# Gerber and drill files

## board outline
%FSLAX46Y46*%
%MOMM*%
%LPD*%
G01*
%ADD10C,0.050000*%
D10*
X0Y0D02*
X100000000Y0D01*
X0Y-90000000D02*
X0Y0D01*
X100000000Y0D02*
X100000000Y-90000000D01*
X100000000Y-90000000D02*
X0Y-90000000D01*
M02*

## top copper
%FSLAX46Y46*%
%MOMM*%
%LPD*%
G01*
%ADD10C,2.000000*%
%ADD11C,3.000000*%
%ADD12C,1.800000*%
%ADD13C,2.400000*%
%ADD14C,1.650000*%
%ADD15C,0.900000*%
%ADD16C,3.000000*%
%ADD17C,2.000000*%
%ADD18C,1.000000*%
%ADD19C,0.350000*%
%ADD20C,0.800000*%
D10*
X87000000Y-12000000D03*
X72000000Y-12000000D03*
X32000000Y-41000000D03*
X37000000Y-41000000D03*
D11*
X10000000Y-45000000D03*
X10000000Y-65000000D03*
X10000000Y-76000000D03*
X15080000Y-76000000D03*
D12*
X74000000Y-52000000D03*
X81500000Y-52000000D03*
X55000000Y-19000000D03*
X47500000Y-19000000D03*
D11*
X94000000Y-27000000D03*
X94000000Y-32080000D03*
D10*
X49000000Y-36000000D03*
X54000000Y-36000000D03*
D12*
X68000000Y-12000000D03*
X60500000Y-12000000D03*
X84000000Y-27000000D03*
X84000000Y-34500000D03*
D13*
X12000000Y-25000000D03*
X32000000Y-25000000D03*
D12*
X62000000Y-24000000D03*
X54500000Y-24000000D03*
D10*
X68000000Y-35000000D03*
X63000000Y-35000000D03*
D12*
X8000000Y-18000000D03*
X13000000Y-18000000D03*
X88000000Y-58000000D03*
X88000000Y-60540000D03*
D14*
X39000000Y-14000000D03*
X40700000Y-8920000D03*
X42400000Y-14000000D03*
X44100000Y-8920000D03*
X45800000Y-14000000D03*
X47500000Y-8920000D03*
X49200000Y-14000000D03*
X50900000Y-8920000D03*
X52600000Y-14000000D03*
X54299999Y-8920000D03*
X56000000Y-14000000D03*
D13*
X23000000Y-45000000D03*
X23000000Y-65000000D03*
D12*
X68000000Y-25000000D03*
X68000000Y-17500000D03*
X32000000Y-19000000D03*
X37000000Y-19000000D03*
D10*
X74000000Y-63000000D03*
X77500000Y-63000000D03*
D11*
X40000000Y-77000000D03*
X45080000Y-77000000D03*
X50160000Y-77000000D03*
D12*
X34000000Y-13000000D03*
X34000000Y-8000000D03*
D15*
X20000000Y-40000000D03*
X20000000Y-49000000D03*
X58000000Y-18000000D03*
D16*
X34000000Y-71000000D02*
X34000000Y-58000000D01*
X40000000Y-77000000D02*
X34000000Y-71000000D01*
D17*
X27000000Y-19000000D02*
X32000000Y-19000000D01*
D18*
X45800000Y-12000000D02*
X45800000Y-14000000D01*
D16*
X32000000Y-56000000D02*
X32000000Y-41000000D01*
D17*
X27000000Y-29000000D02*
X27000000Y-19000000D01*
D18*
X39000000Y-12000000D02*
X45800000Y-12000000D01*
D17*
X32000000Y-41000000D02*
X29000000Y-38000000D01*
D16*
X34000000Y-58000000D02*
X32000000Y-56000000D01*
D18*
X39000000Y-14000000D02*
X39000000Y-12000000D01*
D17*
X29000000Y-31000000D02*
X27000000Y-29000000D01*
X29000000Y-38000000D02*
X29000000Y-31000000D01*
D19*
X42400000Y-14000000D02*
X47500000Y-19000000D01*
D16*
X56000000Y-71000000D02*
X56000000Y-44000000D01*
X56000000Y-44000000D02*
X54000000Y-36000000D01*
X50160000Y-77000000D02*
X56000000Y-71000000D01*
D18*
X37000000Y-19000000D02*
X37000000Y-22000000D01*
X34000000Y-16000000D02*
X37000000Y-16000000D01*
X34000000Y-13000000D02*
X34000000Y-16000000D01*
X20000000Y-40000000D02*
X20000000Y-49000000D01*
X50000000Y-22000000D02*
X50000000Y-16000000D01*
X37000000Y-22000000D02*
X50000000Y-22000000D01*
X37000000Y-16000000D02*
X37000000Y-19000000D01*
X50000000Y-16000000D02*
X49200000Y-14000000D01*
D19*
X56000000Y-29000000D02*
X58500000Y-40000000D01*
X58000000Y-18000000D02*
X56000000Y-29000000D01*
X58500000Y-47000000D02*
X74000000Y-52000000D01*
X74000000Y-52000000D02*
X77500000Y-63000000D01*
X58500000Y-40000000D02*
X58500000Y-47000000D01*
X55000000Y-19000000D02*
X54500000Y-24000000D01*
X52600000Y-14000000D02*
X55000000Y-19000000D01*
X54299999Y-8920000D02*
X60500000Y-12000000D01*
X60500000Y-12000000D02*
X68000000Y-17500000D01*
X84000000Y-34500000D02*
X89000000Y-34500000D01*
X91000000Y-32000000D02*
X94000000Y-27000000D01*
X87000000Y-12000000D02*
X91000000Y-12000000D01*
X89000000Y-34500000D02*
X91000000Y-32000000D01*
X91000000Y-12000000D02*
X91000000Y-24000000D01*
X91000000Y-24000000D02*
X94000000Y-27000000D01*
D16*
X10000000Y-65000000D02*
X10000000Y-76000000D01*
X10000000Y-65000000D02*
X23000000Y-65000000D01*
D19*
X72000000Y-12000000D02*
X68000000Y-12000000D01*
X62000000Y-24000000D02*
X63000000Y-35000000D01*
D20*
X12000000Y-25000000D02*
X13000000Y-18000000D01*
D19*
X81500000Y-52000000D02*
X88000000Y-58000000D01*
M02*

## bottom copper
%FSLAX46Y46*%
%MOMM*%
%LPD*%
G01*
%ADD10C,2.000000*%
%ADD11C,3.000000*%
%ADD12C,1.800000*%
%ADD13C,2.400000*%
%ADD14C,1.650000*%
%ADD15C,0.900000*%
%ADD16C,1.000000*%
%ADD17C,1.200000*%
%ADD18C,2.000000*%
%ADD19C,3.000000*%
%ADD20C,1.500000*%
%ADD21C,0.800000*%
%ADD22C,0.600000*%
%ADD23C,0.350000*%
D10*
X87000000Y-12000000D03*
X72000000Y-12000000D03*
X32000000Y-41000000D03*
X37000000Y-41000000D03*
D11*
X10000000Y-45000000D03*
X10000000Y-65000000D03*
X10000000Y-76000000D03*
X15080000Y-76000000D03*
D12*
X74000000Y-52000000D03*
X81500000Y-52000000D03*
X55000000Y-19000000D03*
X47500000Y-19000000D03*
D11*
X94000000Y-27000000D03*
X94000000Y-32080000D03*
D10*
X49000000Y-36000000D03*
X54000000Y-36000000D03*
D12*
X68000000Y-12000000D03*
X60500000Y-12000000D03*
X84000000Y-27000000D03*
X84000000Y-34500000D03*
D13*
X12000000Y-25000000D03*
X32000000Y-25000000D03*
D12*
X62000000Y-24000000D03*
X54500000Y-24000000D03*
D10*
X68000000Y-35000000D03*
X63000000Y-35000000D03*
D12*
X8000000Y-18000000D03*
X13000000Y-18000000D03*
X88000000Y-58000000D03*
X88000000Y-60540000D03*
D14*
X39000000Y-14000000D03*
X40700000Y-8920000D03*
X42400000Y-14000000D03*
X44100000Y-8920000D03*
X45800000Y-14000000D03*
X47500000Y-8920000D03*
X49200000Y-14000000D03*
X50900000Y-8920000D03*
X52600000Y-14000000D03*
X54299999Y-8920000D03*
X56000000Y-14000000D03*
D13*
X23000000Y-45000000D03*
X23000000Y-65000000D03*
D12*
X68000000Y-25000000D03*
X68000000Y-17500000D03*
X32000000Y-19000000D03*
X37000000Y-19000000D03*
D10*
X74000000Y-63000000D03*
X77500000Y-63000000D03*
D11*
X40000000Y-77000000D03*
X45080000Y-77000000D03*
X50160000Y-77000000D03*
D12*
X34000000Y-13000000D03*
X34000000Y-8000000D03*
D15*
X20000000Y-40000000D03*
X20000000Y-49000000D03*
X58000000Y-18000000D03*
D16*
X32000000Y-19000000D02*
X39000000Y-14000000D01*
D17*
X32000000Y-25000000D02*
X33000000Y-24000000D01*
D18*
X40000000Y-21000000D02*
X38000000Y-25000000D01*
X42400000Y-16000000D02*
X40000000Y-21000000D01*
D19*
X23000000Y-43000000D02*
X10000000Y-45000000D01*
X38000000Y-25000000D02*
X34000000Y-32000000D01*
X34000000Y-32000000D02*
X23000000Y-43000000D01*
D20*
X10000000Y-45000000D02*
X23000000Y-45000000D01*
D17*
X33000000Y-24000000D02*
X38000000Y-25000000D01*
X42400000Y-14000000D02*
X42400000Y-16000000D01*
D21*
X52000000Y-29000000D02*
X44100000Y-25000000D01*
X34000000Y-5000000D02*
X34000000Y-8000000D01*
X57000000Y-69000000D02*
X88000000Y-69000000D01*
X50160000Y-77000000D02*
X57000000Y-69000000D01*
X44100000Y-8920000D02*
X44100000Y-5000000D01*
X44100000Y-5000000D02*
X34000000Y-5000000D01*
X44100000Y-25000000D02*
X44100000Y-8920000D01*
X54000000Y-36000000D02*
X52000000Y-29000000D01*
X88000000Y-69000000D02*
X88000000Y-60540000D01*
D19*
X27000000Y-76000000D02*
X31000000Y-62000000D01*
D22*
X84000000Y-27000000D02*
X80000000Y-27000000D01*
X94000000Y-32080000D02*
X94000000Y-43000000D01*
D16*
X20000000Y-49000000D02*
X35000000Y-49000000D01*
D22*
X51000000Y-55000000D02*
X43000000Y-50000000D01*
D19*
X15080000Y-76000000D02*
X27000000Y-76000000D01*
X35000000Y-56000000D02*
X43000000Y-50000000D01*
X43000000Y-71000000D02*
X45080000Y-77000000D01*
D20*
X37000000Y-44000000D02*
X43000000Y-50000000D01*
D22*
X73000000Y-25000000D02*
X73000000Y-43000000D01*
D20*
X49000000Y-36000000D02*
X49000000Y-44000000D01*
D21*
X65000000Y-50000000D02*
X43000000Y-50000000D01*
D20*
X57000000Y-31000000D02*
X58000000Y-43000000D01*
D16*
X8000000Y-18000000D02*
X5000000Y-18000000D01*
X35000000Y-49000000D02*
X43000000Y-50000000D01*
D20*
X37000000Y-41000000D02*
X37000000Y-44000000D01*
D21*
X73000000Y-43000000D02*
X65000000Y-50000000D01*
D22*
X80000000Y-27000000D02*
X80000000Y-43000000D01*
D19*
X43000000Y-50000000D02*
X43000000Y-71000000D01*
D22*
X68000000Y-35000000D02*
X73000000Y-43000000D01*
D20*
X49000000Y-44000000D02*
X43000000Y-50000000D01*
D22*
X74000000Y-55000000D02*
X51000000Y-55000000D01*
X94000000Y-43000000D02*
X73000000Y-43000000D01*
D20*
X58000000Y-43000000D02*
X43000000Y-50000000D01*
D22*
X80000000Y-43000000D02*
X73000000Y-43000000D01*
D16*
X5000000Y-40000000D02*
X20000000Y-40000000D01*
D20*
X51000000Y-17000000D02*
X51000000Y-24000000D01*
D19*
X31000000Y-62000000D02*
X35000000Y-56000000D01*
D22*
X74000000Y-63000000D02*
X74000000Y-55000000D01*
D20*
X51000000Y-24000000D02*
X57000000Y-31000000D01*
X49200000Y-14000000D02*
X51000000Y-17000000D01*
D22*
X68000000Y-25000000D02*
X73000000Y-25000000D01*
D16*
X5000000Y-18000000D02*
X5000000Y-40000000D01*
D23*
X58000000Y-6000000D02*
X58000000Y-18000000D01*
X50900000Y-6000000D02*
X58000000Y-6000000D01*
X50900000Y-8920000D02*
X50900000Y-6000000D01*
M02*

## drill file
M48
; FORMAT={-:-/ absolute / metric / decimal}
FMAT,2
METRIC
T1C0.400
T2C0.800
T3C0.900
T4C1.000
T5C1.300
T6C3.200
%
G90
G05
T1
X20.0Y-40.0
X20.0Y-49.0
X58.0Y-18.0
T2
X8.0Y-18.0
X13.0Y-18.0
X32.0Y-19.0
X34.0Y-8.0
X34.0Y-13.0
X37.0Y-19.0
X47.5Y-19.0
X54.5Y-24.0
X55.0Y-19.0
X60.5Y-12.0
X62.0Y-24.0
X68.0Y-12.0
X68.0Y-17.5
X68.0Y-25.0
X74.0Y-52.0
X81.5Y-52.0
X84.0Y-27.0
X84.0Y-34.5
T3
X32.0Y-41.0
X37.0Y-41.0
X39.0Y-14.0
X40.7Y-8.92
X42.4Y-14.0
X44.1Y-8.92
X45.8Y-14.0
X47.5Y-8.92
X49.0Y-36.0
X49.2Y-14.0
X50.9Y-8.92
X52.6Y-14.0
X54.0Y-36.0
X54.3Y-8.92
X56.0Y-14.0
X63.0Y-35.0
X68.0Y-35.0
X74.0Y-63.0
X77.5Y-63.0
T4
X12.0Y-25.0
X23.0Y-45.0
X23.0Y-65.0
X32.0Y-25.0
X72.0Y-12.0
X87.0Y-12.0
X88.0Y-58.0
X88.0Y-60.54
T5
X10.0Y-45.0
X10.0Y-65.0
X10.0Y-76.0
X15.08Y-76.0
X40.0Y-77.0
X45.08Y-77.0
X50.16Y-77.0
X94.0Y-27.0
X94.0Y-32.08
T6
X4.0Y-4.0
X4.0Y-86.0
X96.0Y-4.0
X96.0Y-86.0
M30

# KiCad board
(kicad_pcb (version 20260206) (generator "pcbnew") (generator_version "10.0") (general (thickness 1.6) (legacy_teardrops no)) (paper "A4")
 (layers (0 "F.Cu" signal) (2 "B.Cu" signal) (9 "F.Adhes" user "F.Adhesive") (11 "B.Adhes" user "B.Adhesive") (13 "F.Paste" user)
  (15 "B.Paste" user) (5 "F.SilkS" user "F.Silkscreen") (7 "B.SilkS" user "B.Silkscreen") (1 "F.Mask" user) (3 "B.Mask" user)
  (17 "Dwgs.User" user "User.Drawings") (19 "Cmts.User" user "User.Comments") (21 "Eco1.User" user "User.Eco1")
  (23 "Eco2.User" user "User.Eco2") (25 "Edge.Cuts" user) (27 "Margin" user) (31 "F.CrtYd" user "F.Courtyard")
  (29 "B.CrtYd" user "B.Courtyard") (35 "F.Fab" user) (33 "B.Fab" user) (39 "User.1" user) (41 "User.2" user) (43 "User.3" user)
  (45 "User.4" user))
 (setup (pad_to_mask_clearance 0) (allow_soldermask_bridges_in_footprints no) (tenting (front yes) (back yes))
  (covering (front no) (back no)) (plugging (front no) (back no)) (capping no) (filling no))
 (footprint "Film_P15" (layer "F.Cu") (at 87 12 180)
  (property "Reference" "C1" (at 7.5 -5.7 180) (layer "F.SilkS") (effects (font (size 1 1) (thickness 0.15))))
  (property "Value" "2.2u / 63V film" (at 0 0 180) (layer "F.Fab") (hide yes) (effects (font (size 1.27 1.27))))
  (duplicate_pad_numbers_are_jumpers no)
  (pad "1" thru_hole circle (at 0 0 180) (size 2 2) (drill 1) (layers "*.Cu" "*.Mask") (remove_unused_layers no) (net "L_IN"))
  (pad "2" thru_hole circle (at 15 0 180) (size 2 2) (drill 1) (layers "*.Cu" "*.Mask") (remove_unused_layers no) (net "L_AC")))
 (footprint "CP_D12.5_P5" (layer "F.Cu") (at 32 41)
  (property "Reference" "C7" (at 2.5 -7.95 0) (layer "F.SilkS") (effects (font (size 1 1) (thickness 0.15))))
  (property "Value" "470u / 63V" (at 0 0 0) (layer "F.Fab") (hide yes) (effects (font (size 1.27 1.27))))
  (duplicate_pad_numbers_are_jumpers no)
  (pad "1" thru_hole circle (at 0 0) (size 2 2) (drill 0.9) (layers "*.Cu" "*.Mask") (remove_unused_layers no) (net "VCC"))
  (pad "2" thru_hole circle (at 5 0) (size 2 2) (drill 0.9) (layers "*.Cu" "*.Mask") (remove_unused_layers no) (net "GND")))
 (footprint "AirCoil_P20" (layer "F.Cu") (at 10 45 -90)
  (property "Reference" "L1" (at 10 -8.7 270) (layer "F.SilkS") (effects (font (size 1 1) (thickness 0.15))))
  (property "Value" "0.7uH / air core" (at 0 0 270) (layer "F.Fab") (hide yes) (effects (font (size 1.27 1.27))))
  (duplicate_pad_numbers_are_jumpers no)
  (pad "1" thru_hole circle (at 0 0 270) (size 3 3) (drill 1.3) (layers "*.Cu" "*.Mask") (remove_unused_layers no) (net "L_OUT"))
  (pad "2" thru_hole circle (at 20 0 270) (size 3 3) (drill 1.3) (layers "*.Cu" "*.Mask") (remove_unused_layers no) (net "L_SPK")))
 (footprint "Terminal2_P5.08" (layer "F.Cu") (at 10 76)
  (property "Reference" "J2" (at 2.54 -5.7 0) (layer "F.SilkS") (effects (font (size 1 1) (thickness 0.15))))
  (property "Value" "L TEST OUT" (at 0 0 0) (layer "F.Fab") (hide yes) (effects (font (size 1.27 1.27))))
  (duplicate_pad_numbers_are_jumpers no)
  (pad "1" thru_hole circle (at 0 0) (size 3 3) (drill 1.3) (layers "*.Cu" "*.Mask") (remove_unused_layers no) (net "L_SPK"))
  (pad "2" thru_hole circle (at 5.08 0) (size 3 3) (drill 1.3) (layers "*.Cu" "*.Mask") (remove_unused_layers no) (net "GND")))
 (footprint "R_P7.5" (layer "F.Cu") (at 74 52)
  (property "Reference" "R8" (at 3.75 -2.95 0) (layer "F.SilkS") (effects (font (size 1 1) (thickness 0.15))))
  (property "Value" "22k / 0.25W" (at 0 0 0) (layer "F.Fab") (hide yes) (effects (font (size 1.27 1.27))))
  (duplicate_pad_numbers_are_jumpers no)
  (pad "1" thru_hole circle (at 0 0) (size 1.8 1.8) (drill 0.8) (layers "*.Cu" "*.Mask") (remove_unused_layers no) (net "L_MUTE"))
  (pad "2" thru_hole circle (at 7.5 0) (size 1.8 1.8) (drill 0.8) (layers "*.Cu" "*.Mask") (remove_unused_layers no) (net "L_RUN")))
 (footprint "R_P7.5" (layer "F.Cu") (at 55 19 180)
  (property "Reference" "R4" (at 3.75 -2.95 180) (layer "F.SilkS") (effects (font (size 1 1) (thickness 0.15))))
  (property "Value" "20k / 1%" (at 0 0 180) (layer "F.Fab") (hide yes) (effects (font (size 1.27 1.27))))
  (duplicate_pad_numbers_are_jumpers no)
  (pad "1" thru_hole circle (at 0 0 180) (size 1.8 1.8) (drill 0.8) (layers "*.Cu" "*.Mask") (remove_unused_layers no) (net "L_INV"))
  (pad "2" thru_hole circle (at 7.5 0 180) (size 1.8 1.8) (drill 0.8) (layers "*.Cu" "*.Mask") (remove_unused_layers no) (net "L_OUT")))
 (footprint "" (layer "F.Cu") (at 4 86)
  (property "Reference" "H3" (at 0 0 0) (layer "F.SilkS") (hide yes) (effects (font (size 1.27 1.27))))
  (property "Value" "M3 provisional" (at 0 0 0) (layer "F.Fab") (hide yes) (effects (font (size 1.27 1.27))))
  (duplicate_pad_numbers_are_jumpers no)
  (pad "" np_thru_hole circle (at 0 0) (size 3.2 3.2) (drill 3.2) (layers "*.Cu" "*.Mask")))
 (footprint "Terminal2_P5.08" (layer "F.Cu") (at 94 27 -90)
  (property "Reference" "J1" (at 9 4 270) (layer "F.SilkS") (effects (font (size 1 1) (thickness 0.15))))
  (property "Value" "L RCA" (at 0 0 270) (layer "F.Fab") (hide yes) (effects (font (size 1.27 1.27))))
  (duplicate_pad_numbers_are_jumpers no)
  (pad "1" thru_hole circle (at 0 0 270) (size 3 3) (drill 1.3) (layers "*.Cu" "*.Mask") (remove_unused_layers no) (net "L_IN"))
  (pad "2" thru_hole circle (at 5.08 0 270) (size 3 3) (drill 1.3) (layers "*.Cu" "*.Mask") (remove_unused_layers no) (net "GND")))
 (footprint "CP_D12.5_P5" (layer "F.Cu") (at 49 36)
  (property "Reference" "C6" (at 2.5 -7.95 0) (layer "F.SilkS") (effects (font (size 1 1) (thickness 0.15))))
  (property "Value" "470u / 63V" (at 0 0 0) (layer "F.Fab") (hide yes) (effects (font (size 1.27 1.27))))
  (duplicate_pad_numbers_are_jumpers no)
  (pad "1" thru_hole circle (at 0 0) (size 2 2) (drill 0.9) (layers "*.Cu" "*.Mask") (remove_unused_layers no) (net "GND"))
  (pad "2" thru_hole circle (at 5 0) (size 2 2) (drill 0.9) (layers "*.Cu" "*.Mask") (remove_unused_layers no) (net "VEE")))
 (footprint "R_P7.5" (layer "F.Cu") (at 68 12 180)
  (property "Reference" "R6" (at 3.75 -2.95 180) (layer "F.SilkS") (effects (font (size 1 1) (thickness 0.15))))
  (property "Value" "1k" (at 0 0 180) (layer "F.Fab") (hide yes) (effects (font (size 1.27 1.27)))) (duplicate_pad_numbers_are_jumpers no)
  (pad "1" thru_hole circle (at 0 0 180) (size 1.8 1.8) (drill 0.8) (layers "*.Cu" "*.Mask") (remove_unused_layers no) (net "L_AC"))
  (pad "2" thru_hole circle (at 7.5 0 180) (size 1.8 1.8) (drill 0.8) (layers "*.Cu" "*.Mask") (remove_unused_layers no) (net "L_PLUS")))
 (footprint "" (layer "F.Cu") (at 4 4)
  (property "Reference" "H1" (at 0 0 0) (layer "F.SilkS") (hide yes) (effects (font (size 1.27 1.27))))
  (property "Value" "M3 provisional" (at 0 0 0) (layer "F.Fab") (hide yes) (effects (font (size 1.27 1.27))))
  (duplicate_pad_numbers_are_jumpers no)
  (pad "" np_thru_hole circle (at 0 0) (size 3.2 3.2) (drill 3.2) (layers "*.Cu" "*.Mask")))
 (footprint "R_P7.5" (layer "F.Cu") (at 84 27 -90)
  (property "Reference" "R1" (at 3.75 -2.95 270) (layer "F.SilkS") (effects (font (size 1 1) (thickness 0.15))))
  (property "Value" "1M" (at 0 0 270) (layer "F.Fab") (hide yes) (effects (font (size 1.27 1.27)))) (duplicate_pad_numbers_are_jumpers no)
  (pad "1" thru_hole circle (at 0 0 270) (size 1.8 1.8) (drill 0.8) (layers "*.Cu" "*.Mask") (remove_unused_layers no) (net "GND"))
  (pad "2" thru_hole circle (at 7.5 0 270) (size 1.8 1.8) (drill 0.8) (layers "*.Cu" "*.Mask") (remove_unused_layers no) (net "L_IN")))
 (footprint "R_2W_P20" (layer "F.Cu") (at 12 25)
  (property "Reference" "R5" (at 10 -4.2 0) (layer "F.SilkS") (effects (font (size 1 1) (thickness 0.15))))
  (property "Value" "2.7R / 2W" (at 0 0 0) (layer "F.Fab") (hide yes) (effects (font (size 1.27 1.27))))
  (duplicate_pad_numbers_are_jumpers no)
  (pad "1" thru_hole circle (at 0 0) (size 2.4 2.4) (drill 1) (layers "*.Cu" "*.Mask") (remove_unused_layers no) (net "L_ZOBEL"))
  (pad "2" thru_hole circle (at 20 0) (size 2.4 2.4) (drill 1) (layers "*.Cu" "*.Mask") (remove_unused_layers no) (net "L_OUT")))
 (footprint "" (layer "F.Cu") (at 96 4)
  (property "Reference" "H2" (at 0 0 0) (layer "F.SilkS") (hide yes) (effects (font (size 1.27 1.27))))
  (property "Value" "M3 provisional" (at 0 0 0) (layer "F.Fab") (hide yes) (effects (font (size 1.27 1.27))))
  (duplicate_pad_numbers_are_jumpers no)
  (pad "" np_thru_hole circle (at 0 0) (size 3.2 3.2) (drill 3.2) (layers "*.Cu" "*.Mask")))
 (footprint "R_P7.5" (layer "F.Cu") (at 62 24 180)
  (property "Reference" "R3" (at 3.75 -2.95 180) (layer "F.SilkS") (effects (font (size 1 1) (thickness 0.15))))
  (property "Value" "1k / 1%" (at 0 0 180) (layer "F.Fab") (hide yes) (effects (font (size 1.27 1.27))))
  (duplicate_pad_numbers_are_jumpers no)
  (pad "1" thru_hole circle (at 0 0 180) (size 1.8 1.8) (drill 0.8) (layers "*.Cu" "*.Mask") (remove_unused_layers no) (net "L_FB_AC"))
  (pad "2" thru_hole circle (at 7.5 0 180) (size 1.8 1.8) (drill 0.8) (layers "*.Cu" "*.Mask") (remove_unused_layers no) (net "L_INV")))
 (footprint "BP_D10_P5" (layer "F.Cu") (at 68 35 180)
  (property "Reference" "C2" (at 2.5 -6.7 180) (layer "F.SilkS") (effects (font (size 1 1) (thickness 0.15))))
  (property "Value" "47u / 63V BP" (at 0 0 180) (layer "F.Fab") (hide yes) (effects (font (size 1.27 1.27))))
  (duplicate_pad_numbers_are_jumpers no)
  (pad "1" thru_hole circle (at 0 0 180) (size 2 2) (drill 0.9) (layers "*.Cu" "*.Mask") (remove_unused_layers no) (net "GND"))
  (pad "2" thru_hole circle (at 5 0 180) (size 2 2) (drill 0.9) (layers "*.Cu" "*.Mask") (remove_unused_layers no) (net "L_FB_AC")))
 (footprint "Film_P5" (layer "F.Cu") (at 8 18)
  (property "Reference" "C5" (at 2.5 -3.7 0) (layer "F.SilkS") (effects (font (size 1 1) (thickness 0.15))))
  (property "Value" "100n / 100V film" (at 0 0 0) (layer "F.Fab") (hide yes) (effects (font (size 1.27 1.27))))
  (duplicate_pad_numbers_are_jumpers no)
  (pad "1" thru_hole circle (at 0 0) (size 1.8 1.8) (drill 0.8) (layers "*.Cu" "*.Mask") (remove_unused_layers no) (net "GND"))
  (pad "2" thru_hole circle (at 5 0) (size 1.8 1.8) (drill 0.8) (layers "*.Cu" "*.Mask") (remove_unused_layers no) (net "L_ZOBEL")))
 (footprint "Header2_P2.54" (layer "F.Cu") (at 88 58 -90)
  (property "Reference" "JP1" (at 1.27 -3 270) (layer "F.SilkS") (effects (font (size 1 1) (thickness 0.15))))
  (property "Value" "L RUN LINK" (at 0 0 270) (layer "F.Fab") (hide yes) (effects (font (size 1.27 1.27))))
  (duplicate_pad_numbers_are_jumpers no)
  (pad "1" thru_hole circle (at 0 0 270) (size 1.8 1.8) (drill 1) (layers "*.Cu" "*.Mask") (remove_unused_layers no) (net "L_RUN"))
  (pad "2" thru_hole circle (at 2.54 0 270) (size 1.8 1.8) (drill 1) (layers "*.Cu" "*.Mask") (remove_unused_layers no) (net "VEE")))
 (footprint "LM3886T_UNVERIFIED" (layer "F.Cu") (at 39 14)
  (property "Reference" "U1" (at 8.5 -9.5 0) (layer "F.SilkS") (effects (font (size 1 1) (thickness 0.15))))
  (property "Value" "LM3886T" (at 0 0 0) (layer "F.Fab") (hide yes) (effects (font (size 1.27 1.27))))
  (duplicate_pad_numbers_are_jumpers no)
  (pad "1" thru_hole circle (at 0 0) (size 1.65 1.65) (drill 0.9) (layers "*.Cu" "*.Mask") (remove_unused_layers no) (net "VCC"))
  (pad "2" thru_hole circle (at 1.7 -5.08) (size 1.65 1.65) (drill 0.9) (layers "*.Cu" "*.Mask") (remove_unused_layers no)
   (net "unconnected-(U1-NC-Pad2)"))
  (pad "3" thru_hole circle (at 3.4 0) (size 1.65 1.65) (drill 0.9) (layers "*.Cu" "*.Mask") (remove_unused_layers no) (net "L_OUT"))
  (pad "4" thru_hole circle (at 5.1 -5.08) (size 1.65 1.65) (drill 0.9) (layers "*.Cu" "*.Mask") (remove_unused_layers no) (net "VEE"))
  (pad "5" thru_hole circle (at 6.8 0) (size 1.65 1.65) (drill 0.9) (layers "*.Cu" "*.Mask") (remove_unused_layers no) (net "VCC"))
  (pad "6" thru_hole circle (at 8.5 -5.08) (size 1.65 1.65) (drill 0.9) (layers "*.Cu" "*.Mask") (remove_unused_layers no)
   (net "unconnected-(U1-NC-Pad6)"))
  (pad "7" thru_hole circle (at 10.2 0) (size 1.65 1.65) (drill 0.9) (layers "*.Cu" "*.Mask") (remove_unused_layers no) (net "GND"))
  (pad "8" thru_hole circle (at 11.9 -5.08) (size 1.65 1.65) (drill 0.9) (layers "*.Cu" "*.Mask") (remove_unused_layers no) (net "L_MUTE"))
  (pad "9" thru_hole circle (at 13.6 0) (size 1.65 1.65) (drill 0.9) (layers "*.Cu" "*.Mask") (remove_unused_layers no) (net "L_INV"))
  (pad "10" thru_hole circle (at 15.299999 -5.08) (size 1.65 1.65) (drill 0.9) (layers "*.Cu" "*.Mask") (remove_unused_layers no)
   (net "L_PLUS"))
  (pad "11" thru_hole circle (at 17 0) (size 1.65 1.65) (drill 0.9) (layers "*.Cu" "*.Mask") (remove_unused_layers no)
   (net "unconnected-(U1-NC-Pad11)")))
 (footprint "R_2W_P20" (layer "F.Cu") (at 23 45 -90)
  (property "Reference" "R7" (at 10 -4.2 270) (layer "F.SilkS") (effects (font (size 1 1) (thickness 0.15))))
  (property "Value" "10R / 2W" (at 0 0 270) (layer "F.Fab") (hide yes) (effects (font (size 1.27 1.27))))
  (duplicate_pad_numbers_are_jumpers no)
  (pad "1" thru_hole circle (at 0 0 270) (size 2.4 2.4) (drill 1) (layers "*.Cu" "*.Mask") (remove_unused_layers no) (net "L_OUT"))
  (pad "2" thru_hole circle (at 20 0 270) (size 2.4 2.4) (drill 1) (layers "*.Cu" "*.Mask") (remove_unused_layers no) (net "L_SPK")))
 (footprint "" (layer "F.Cu") (at 96 86)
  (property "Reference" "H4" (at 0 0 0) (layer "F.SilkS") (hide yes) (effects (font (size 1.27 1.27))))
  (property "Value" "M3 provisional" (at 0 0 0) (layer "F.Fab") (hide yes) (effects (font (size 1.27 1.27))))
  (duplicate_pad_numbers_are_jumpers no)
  (pad "" np_thru_hole circle (at 0 0) (size 3.2 3.2) (drill 3.2) (layers "*.Cu" "*.Mask")))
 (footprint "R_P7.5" (layer "F.Cu") (at 68 25 90)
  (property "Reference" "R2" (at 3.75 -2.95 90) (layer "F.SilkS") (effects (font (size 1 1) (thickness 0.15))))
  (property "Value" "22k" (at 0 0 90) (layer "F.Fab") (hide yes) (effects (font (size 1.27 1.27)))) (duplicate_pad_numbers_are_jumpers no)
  (pad "1" thru_hole circle (at 0 0 90) (size 1.8 1.8) (drill 0.8) (layers "*.Cu" "*.Mask") (remove_unused_layers no) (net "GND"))
  (pad "2" thru_hole circle (at 7.5 0 90) (size 1.8 1.8) (drill 0.8) (layers "*.Cu" "*.Mask") (remove_unused_layers no) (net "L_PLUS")))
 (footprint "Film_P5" (layer "F.Cu") (at 32 19)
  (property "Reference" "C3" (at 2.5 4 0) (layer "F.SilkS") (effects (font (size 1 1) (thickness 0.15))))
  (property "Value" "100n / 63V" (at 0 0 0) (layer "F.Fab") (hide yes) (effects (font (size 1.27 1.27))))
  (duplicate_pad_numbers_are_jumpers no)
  (pad "1" thru_hole circle (at 0 0) (size 1.8 1.8) (drill 0.8) (layers "*.Cu" "*.Mask") (remove_unused_layers no) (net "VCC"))
  (pad "2" thru_hole circle (at 5 0) (size 1.8 1.8) (drill 0.8) (layers "*.Cu" "*.Mask") (remove_unused_layers no) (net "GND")))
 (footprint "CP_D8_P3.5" (layer "F.Cu") (at 74 63)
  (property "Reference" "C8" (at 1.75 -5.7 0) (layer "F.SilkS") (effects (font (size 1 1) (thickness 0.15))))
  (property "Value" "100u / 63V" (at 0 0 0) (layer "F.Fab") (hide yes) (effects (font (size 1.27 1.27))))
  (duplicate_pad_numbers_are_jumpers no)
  (pad "1" thru_hole circle (at 0 0) (size 2 2) (drill 0.9) (layers "*.Cu" "*.Mask") (remove_unused_layers no) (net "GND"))
  (pad "2" thru_hole circle (at 3.5 0) (size 2 2) (drill 0.9) (layers "*.Cu" "*.Mask") (remove_unused_layers no) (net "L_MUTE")))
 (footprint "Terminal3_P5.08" (layer "F.Cu") (at 40 77)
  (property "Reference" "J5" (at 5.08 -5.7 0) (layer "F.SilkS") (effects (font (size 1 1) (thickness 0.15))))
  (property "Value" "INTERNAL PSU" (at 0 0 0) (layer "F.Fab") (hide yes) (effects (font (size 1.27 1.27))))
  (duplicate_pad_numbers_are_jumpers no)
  (pad "1" thru_hole circle (at 0 0) (size 3 3) (drill 1.3) (layers "*.Cu" "*.Mask") (remove_unused_layers no) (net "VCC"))
  (pad "2" thru_hole circle (at 5.08 0) (size 3 3) (drill 1.3) (layers "*.Cu" "*.Mask") (remove_unused_layers no) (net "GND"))
  (pad "3" thru_hole circle (at 10.16 0) (size 3 3) (drill 1.3) (layers "*.Cu" "*.Mask") (remove_unused_layers no) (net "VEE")))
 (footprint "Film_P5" (layer "F.Cu") (at 34 13 90)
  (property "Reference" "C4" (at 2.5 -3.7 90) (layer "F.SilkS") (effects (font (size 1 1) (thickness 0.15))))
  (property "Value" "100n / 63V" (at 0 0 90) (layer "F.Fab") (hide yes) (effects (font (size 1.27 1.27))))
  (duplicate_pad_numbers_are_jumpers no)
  (pad "1" thru_hole circle (at 0 0 90) (size 1.8 1.8) (drill 0.8) (layers "*.Cu" "*.Mask") (remove_unused_layers no) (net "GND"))
  (pad "2" thru_hole circle (at 5 0 90) (size 1.8 1.8) (drill 0.8) (layers "*.Cu" "*.Mask") (remove_unused_layers no) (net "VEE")))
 (gr_line (start 0 0) (end 100 0) (stroke (width 0.05) (type default)) (layer "Edge.Cuts"))
 (gr_line (start 0 90) (end 0 0) (stroke (width 0.05) (type default)) (layer "Edge.Cuts"))
 (gr_line (start 100 0) (end 100 90) (stroke (width 0.05) (type default)) (layer "Edge.Cuts"))
 (gr_line (start 100 90) (end 0 90) (stroke (width 0.05) (type default)) (layer "Edge.Cuts"))
 (segment (start 34 71) (end 34 58) (width 3) (layer "F.Cu") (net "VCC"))
 (segment (start 40 77) (end 34 71) (width 3) (layer "F.Cu") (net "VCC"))
 (segment (start 27 19) (end 32 19) (width 2) (layer "F.Cu") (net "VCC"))
 (segment (start 45.8 12) (end 45.8 14) (width 1) (layer "F.Cu") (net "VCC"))
 (segment (start 32 56) (end 32 41) (width 3) (layer "F.Cu") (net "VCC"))
 (segment (start 27 29) (end 27 19) (width 2) (layer "F.Cu") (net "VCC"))
 (segment (start 39 12) (end 45.8 12) (width 1) (layer "F.Cu") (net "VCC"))
 (segment (start 32 41) (end 29 38) (width 2) (layer "F.Cu") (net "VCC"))
 (segment (start 34 58) (end 32 56) (width 3) (layer "F.Cu") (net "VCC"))
 (segment (start 39 14) (end 39 12) (width 1) (layer "F.Cu") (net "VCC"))
 (segment (start 29 31) (end 27 29) (width 2) (layer "F.Cu") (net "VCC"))
 (segment (start 29 38) (end 29 31) (width 2) (layer "F.Cu") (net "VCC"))
 (segment (start 32 19) (end 39 14) (width 1) (layer "B.Cu") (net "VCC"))
 (segment (start 42.4 14) (end 47.5 19) (width 0.35) (layer "F.Cu") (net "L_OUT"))
 (segment (start 32 25) (end 33 24) (width 1.2) (layer "B.Cu") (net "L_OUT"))
 (segment (start 40 21) (end 38 25) (width 2) (layer "B.Cu") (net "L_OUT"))
 (segment (start 42.4 16) (end 40 21) (width 2) (layer "B.Cu") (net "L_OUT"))
 (segment (start 23 43) (end 10 45) (width 3) (layer "B.Cu") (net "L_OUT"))
 (segment (start 38 25) (end 34 32) (width 3) (layer "B.Cu") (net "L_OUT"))
 (segment (start 34 32) (end 23 43) (width 3) (layer "B.Cu") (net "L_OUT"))
 (segment (start 10 45) (end 23 45) (width 1.5) (layer "B.Cu") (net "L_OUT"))
 (segment (start 33 24) (end 38 25) (width 1.2) (layer "B.Cu") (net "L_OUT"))
 (segment (start 42.4 14) (end 42.4 16) (width 1.2) (layer "B.Cu") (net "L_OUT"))
 (segment (start 56 71) (end 56 44) (width 3) (layer "F.Cu") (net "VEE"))
 (segment (start 56 44) (end 54 36) (width 3) (layer "F.Cu") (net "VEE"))
 (segment (start 50.16 77) (end 56 71) (width 3) (layer "F.Cu") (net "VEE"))
 (segment (start 52 29) (end 44.1 25) (width 0.8) (layer "B.Cu") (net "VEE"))
 (segment (start 34 5) (end 34 8) (width 0.8) (layer "B.Cu") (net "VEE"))
 (segment (start 57 69) (end 88 69) (width 0.8) (layer "B.Cu") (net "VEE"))
 (segment (start 50.16 77) (end 57 69) (width 0.8) (layer "B.Cu") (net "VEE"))
 (segment (start 44.1 8.92) (end 44.1 5) (width 0.8) (layer "B.Cu") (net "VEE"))
 (segment (start 44.1 5) (end 34 5) (width 0.8) (layer "B.Cu") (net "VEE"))
 (segment (start 44.1 25) (end 44.1 8.92) (width 0.8) (layer "B.Cu") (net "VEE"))
 (segment (start 54 36) (end 52 29) (width 0.8) (layer "B.Cu") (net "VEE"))
 (segment (start 88 69) (end 88 60.54) (width 0.8) (layer "B.Cu") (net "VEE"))
 (segment (start 37 19) (end 37 22) (width 1) (layer "F.Cu") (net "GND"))
 (segment (start 34 16) (end 37 16) (width 1) (layer "F.Cu") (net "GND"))
 (segment (start 34 13) (end 34 16) (width 1) (layer "F.Cu") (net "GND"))
 (segment (start 20 40) (end 20 49) (width 1) (layer "F.Cu") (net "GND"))
 (segment (start 50 22) (end 50 16) (width 1) (layer "F.Cu") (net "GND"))
 (segment (start 37 22) (end 50 22) (width 1) (layer "F.Cu") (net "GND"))
 (segment (start 37 16) (end 37 19) (width 1) (layer "F.Cu") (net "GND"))
 (segment (start 50 16) (end 49.2 14) (width 1) (layer "F.Cu") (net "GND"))
 (via (at 20 40) (size 0.9) (drill 0.4) (layers "F.Cu" "B.Cu") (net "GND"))
 (via (at 20 49) (size 0.9) (drill 0.4) (layers "F.Cu" "B.Cu") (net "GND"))
 (segment (start 27 76) (end 31 62) (width 3) (layer "B.Cu") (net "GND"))
 (segment (start 84 27) (end 80 27) (width 0.6) (layer "B.Cu") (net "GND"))
 (segment (start 94 32.08) (end 94 43) (width 0.6) (layer "B.Cu") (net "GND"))
 (segment (start 20 49) (end 35 49) (width 1) (layer "B.Cu") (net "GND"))
 (segment (start 51 55) (end 43 50) (width 0.6) (layer "B.Cu") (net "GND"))
 (segment (start 15.08 76) (end 27 76) (width 3) (layer "B.Cu") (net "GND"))
 (segment (start 35 56) (end 43 50) (width 3) (layer "B.Cu") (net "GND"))
 (segment (start 43 71) (end 45.08 77) (width 3) (layer "B.Cu") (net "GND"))
 (segment (start 37 44) (end 43 50) (width 1.5) (layer "B.Cu") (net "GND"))
 (segment (start 73 25) (end 73 43) (width 0.6) (layer "B.Cu") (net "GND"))
 (segment (start 49 36) (end 49 44) (width 1.5) (layer "B.Cu") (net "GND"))
 (segment (start 65 50) (end 43 50) (width 0.8) (layer "B.Cu") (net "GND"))
 (segment (start 57 31) (end 58 43) (width 1.5) (layer "B.Cu") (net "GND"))
 (segment (start 8 18) (end 5 18) (width 1) (layer "B.Cu") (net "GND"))
 (segment (start 35 49) (end 43 50) (width 1) (layer "B.Cu") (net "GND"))
 (segment (start 37 41) (end 37 44) (width 1.5) (layer "B.Cu") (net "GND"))
 (segment (start 73 43) (end 65 50) (width 0.8) (layer "B.Cu") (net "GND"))
 (segment (start 80 27) (end 80 43) (width 0.6) (layer "B.Cu") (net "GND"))
 (segment (start 43 50) (end 43 71) (width 3) (layer "B.Cu") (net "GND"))
 (segment (start 68 35) (end 73 43) (width 0.6) (layer "B.Cu") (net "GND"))
 (segment (start 49 44) (end 43 50) (width 1.5) (layer "B.Cu") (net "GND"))
 (segment (start 74 55) (end 51 55) (width 0.6) (layer "B.Cu") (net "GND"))
 (segment (start 94 43) (end 73 43) (width 0.6) (layer "B.Cu") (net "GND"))
 (segment (start 58 43) (end 43 50) (width 1.5) (layer "B.Cu") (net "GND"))
 (segment (start 80 43) (end 73 43) (width 0.6) (layer "B.Cu") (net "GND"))
 (segment (start 5 40) (end 20 40) (width 1) (layer "B.Cu") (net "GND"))
 (segment (start 51 17) (end 51 24) (width 1.5) (layer "B.Cu") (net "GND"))
 (segment (start 31 62) (end 35 56) (width 3) (layer "B.Cu") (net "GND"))
 (segment (start 74 63) (end 74 55) (width 0.6) (layer "B.Cu") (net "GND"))
 (segment (start 51 24) (end 57 31) (width 1.5) (layer "B.Cu") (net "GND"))
 (segment (start 49.2 14) (end 51 17) (width 1.5) (layer "B.Cu") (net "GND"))
 (segment (start 68 25) (end 73 25) (width 0.6) (layer "B.Cu") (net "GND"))
 (segment (start 5 18) (end 5 40) (width 1) (layer "B.Cu") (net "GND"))
 (segment (start 56 29) (end 58.5 40) (width 0.35) (layer "F.Cu") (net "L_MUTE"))
 (segment (start 58 18) (end 56 29) (width 0.35) (layer "F.Cu") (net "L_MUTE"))
 (segment (start 58.5 47) (end 74 52) (width 0.35) (layer "F.Cu") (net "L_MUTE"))
 (segment (start 74 52) (end 77.5 63) (width 0.35) (layer "F.Cu") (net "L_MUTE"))
 (segment (start 58.5 40) (end 58.5 47) (width 0.35) (layer "F.Cu") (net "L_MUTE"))
 (via (at 58 18) (size 0.9) (drill 0.4) (layers "F.Cu" "B.Cu") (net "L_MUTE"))
 (segment (start 58 6) (end 58 18) (width 0.35) (layer "B.Cu") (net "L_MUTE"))
 (segment (start 50.9 6) (end 58 6) (width 0.35) (layer "B.Cu") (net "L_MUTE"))
 (segment (start 50.9 8.92) (end 50.9 6) (width 0.35) (layer "B.Cu") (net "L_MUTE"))
 (segment (start 55 19) (end 54.5 24) (width 0.35) (layer "F.Cu") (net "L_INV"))
 (segment (start 52.6 14) (end 55 19) (width 0.35) (layer "F.Cu") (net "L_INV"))
 (segment (start 54.299999 8.92) (end 60.5 12) (width 0.35) (layer "F.Cu") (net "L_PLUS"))
 (segment (start 60.5 12) (end 68 17.5) (width 0.35) (layer "F.Cu") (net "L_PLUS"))
 (segment (start 84 34.5) (end 89 34.5) (width 0.35) (layer "F.Cu") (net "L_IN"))
 (segment (start 91 32) (end 94 27) (width 0.35) (layer "F.Cu") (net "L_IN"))
 (segment (start 87 12) (end 91 12) (width 0.35) (layer "F.Cu") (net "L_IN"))
 (segment (start 89 34.5) (end 91 32) (width 0.35) (layer "F.Cu") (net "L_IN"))
 (segment (start 91 12) (end 91 24) (width 0.35) (layer "F.Cu") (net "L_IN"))
 (segment (start 91 24) (end 94 27) (width 0.35) (layer "F.Cu") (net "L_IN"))
 (segment (start 10 65) (end 10 76) (width 3) (layer "F.Cu") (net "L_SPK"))
 (segment (start 10 65) (end 23 65) (width 3) (layer "F.Cu") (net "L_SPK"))
 (segment (start 72 12) (end 68 12) (width 0.35) (layer "F.Cu") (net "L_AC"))
 (segment (start 62 24) (end 63 35) (width 0.35) (layer "F.Cu") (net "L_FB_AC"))
 (segment (start 12 25) (end 13 18) (width 0.8) (layer "F.Cu") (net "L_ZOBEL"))
 (segment (start 81.5 52) (end 88 58) (width 0.35) (layer "F.Cu") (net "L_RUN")))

